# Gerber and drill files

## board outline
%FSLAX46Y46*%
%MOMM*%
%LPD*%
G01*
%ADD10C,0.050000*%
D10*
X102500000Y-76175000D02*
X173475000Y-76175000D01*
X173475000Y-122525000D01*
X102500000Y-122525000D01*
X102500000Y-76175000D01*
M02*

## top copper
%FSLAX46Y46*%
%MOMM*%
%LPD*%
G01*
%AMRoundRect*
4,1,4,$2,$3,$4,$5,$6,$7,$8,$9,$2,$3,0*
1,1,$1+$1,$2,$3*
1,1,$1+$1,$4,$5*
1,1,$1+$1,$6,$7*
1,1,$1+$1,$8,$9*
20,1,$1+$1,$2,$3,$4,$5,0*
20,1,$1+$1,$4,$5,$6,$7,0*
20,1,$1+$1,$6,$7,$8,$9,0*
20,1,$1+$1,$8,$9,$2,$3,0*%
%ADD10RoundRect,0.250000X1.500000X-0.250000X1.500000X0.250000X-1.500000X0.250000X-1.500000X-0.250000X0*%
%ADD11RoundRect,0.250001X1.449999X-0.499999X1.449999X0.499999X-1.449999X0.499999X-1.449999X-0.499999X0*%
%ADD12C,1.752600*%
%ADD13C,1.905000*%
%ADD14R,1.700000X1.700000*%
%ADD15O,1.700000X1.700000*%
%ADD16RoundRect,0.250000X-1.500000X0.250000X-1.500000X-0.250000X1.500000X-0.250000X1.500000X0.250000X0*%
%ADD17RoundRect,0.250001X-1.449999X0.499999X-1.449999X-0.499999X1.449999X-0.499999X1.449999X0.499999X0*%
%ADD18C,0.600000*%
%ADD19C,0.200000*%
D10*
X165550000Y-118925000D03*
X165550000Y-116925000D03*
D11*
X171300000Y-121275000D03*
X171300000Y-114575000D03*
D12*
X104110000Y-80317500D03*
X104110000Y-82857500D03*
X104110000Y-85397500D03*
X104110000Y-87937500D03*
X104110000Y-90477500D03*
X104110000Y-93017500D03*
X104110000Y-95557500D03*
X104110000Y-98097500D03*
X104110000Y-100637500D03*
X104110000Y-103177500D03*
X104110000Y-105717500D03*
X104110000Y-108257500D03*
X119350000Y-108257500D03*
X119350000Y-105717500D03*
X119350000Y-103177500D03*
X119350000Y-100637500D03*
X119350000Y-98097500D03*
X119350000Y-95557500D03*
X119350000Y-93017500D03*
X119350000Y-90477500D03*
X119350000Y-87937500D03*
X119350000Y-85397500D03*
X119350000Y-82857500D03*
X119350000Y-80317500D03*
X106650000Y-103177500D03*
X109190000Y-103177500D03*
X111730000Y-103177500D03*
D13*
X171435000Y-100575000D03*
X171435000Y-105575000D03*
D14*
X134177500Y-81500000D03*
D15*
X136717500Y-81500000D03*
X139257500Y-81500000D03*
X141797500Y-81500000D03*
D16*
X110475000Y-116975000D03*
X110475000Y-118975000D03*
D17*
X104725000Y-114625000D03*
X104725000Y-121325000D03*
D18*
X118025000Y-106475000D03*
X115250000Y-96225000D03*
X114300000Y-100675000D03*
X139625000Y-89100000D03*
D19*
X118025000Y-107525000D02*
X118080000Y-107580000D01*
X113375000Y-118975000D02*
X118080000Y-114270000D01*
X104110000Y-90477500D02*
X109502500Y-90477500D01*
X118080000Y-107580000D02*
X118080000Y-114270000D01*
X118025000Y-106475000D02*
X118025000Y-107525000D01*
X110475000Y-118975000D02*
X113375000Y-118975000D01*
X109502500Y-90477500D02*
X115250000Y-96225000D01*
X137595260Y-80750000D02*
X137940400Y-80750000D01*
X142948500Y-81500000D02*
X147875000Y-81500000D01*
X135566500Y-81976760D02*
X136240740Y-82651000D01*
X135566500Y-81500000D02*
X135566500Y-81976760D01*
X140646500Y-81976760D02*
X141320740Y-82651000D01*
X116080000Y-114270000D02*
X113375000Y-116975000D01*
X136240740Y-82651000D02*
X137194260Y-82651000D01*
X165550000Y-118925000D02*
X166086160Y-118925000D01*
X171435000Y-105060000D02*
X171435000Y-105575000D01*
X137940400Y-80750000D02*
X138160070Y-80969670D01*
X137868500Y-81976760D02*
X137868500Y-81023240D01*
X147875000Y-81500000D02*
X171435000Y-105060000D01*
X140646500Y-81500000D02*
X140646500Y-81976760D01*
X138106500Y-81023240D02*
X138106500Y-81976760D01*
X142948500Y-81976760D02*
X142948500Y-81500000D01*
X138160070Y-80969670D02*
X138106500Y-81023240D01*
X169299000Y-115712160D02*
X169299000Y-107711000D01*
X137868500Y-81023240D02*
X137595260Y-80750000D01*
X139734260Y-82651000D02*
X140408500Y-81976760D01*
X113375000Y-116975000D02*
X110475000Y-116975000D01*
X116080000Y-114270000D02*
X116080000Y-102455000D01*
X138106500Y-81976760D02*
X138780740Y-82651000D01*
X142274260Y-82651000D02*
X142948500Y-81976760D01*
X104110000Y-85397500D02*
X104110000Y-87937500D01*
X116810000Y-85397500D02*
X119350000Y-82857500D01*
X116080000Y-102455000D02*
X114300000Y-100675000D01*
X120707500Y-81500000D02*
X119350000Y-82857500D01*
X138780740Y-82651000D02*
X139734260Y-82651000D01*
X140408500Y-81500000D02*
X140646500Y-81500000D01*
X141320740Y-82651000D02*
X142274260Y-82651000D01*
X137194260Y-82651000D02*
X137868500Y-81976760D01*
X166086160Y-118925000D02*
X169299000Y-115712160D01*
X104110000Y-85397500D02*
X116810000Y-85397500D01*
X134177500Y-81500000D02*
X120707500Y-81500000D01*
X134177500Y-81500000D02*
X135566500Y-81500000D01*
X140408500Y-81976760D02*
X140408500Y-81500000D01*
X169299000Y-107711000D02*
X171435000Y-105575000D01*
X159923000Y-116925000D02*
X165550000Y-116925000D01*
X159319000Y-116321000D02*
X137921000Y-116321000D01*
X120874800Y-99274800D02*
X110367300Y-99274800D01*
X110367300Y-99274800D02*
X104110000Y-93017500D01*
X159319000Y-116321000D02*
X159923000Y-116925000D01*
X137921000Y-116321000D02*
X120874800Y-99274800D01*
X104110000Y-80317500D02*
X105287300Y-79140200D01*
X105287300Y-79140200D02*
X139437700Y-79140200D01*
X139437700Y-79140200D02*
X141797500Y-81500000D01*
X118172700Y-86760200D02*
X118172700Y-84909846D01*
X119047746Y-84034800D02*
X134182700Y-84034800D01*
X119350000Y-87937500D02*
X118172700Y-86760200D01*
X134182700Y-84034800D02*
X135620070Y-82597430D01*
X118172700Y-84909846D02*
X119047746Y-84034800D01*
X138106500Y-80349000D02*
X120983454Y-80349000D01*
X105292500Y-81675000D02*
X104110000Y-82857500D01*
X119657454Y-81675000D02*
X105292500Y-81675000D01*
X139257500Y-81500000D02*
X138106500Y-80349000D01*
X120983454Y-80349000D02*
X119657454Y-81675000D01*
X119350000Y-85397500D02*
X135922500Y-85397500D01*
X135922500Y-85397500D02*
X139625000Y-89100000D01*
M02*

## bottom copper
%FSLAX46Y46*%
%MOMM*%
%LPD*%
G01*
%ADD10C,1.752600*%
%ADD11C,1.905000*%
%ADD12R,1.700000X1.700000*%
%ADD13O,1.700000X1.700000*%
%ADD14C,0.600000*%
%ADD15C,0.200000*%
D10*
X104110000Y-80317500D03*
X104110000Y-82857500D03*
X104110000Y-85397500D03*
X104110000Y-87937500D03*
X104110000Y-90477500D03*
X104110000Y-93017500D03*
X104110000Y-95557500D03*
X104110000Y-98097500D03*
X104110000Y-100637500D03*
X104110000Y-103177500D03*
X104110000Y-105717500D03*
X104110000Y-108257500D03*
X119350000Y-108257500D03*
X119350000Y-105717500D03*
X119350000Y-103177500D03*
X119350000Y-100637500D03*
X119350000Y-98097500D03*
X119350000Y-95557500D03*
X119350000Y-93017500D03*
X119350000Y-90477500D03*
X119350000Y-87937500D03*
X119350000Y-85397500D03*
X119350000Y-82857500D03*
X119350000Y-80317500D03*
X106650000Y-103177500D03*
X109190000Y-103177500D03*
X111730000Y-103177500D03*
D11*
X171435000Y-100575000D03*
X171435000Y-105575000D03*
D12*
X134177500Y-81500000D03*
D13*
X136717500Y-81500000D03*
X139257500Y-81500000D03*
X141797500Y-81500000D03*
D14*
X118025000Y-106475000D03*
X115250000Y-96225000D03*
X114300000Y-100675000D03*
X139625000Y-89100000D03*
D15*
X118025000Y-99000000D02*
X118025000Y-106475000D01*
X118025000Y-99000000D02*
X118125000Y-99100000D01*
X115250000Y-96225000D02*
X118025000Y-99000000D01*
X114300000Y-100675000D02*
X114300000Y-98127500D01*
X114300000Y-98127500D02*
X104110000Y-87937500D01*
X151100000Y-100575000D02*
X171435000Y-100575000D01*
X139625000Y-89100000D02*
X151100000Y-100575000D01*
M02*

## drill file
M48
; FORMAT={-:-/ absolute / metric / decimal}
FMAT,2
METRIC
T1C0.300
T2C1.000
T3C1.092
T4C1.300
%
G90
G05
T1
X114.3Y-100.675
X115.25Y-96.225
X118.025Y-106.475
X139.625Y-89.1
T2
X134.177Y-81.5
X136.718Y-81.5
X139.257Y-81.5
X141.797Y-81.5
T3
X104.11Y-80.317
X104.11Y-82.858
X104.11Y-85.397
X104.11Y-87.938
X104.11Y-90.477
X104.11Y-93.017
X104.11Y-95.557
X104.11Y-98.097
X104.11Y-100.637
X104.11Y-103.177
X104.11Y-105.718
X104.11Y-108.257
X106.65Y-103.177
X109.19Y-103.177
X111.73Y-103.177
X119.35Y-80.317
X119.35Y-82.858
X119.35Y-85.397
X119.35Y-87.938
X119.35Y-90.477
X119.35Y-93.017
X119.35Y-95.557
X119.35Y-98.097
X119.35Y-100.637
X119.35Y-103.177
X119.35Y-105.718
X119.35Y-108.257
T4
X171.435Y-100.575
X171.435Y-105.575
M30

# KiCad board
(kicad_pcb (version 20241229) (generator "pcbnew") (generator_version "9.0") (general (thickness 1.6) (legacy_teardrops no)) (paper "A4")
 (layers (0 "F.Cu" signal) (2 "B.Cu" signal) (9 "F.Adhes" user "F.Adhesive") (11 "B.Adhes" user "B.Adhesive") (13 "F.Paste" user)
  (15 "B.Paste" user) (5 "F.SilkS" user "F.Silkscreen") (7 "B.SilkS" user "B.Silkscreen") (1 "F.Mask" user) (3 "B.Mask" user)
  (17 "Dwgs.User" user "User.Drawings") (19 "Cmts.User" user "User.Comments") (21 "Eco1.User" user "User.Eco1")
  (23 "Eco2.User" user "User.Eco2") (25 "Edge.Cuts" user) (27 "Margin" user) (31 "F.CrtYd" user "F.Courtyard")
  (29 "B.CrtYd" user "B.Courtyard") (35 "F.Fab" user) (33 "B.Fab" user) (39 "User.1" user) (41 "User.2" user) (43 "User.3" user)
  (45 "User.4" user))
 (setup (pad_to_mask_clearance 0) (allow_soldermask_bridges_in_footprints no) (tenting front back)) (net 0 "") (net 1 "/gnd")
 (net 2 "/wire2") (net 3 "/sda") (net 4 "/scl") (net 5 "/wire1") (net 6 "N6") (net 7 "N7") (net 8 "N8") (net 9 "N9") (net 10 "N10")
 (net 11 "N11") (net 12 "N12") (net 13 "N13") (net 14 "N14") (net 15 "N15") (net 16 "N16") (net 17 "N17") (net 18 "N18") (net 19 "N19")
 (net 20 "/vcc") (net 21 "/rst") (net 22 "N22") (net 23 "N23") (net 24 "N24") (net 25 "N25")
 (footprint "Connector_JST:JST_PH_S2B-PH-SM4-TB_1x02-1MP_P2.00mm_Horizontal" (layer "F.Cu") (at 168.4 117.925 90)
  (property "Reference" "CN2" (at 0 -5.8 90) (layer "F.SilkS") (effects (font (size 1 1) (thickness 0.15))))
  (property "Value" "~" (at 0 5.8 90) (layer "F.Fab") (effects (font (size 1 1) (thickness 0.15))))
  (pad "1" smd roundrect (at -1 -2.85 90) (size 1 3.5) (layers "F.Cu" "F.Mask" "F.Paste") (roundrect_rratio 0.25) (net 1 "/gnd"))
  (pad "2" smd roundrect (at 1 -2.85 90) (size 1 3.5) (layers "F.Cu" "F.Mask" "F.Paste") (roundrect_rratio 0.25) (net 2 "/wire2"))
  (pad "MP" smd roundrect (at -3.35 2.9 90) (size 1.5 3.4) (layers "F.Cu" "F.Mask" "F.Paste") (roundrect_rratio 0.166667))
  (pad "MP" smd roundrect (at 3.35 2.9 90) (size 1.5 3.4) (layers "F.Cu" "F.Mask" "F.Paste") (roundrect_rratio 0.166667)))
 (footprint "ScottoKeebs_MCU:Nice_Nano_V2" (layer "F.Cu") (at 111.73 94.0075)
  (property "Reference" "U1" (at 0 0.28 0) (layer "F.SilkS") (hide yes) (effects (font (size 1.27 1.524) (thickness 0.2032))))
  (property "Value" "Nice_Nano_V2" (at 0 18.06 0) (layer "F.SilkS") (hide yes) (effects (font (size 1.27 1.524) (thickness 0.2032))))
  (pad "1" thru_hole circle (at -7.62 -13.69 270) (size 1.7526 1.7526) (drill 1.0922) (layers "*.Cu" "*.Mask") (remove_unused_layers no)
   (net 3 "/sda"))
  (pad "2" thru_hole circle (at -7.62 -11.15 270) (size 1.7526 1.7526) (drill 1.0922) (layers "*.Cu" "*.Mask") (remove_unused_layers no)
   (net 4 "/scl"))
  (pad "3" thru_hole circle (at -7.62 -8.61 270) (size 1.7526 1.7526) (drill 1.0922) (layers "*.Cu" "*.Mask") (remove_unused_layers no)
   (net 1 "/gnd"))
  (pad "4" thru_hole circle (at -7.62 -6.07 270) (size 1.7526 1.7526) (drill 1.0922) (layers "*.Cu" "*.Mask") (remove_unused_layers no)
   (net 1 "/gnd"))
  (pad "5" thru_hole circle (at -7.62 -3.53 270) (size 1.7526 1.7526) (drill 1.0922) (layers "*.Cu" "*.Mask") (remove_unused_layers no)
   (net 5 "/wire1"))
  (pad "6" thru_hole circle (at -7.62 -0.99 270) (size 1.7526 1.7526) (drill 1.0922) (layers "*.Cu" "*.Mask") (remove_unused_layers no)
   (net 2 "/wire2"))
  (pad "7" thru_hole circle (at -7.62 1.55 270) (size 1.7526 1.7526) (drill 1.0922) (layers "*.Cu" "*.Mask") (remove_unused_layers no)
   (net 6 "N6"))
  (pad "8" thru_hole circle (at -7.62 4.09 270) (size 1.7526 1.7526) (drill 1.0922) (layers "*.Cu" "*.Mask") (remove_unused_layers no)
   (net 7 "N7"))
  (pad "9" thru_hole circle (at -7.62 6.63 270) (size 1.7526 1.7526) (drill 1.0922) (layers "*.Cu" "*.Mask") (remove_unused_layers no)
   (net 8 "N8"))
  (pad "10" thru_hole circle (at -7.62 9.17 270) (size 1.7526 1.7526) (drill 1.0922) (layers "*.Cu" "*.Mask") (remove_unused_layers no)
   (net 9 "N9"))
  (pad "11" thru_hole circle (at -7.62 11.71 270) (size 1.7526 1.7526) (drill 1.0922) (layers "*.Cu" "*.Mask") (remove_unused_layers no)
   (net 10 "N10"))
  (pad "12" thru_hole circle (at -7.62 14.25 270) (size 1.7526 1.7526) (drill 1.0922) (layers "*.Cu" "*.Mask") (remove_unused_layers no)
   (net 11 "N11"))
  (pad "13" thru_hole circle (at 7.62 14.25 270) (size 1.7526 1.7526) (drill 1.0922) (layers "*.Cu" "*.Mask") (remove_unused_layers no)
   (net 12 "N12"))
  (pad "14" thru_hole circle (at 7.62 11.71 270) (size 1.7526 1.7526) (drill 1.0922) (layers "*.Cu" "*.Mask") (remove_unused_layers no)
   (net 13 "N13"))
  (pad "15" thru_hole circle (at 7.62 9.17 270) (size 1.7526 1.7526) (drill 1.0922) (layers "*.Cu" "*.Mask") (remove_unused_layers no)
   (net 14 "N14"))
  (pad "16" thru_hole circle (at 7.62 6.63 270) (size 1.7526 1.7526) (drill 1.0922) (layers "*.Cu" "*.Mask") (remove_unused_layers no)
   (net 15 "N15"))
  (pad "17" thru_hole circle (at 7.62 4.09 270) (size 1.7526 1.7526) (drill 1.0922) (layers "*.Cu" "*.Mask") (remove_unused_layers no)
   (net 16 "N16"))
  (pad "18" thru_hole circle (at 7.62 1.55 270) (size 1.7526 1.7526) (drill 1.0922) (layers "*.Cu" "*.Mask") (remove_unused_layers no)
   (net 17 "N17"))
  (pad "19" thru_hole circle (at 7.62 -0.99 270) (size 1.7526 1.7526) (drill 1.0922) (layers "*.Cu" "*.Mask") (remove_unused_layers no)
   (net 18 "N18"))
  (pad "20" thru_hole circle (at 7.62 -3.53 270) (size 1.7526 1.7526) (drill 1.0922) (layers "*.Cu" "*.Mask") (remove_unused_layers no)
   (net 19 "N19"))
  (pad "21" thru_hole circle (at 7.62 -6.07 270) (size 1.7526 1.7526) (drill 1.0922) (layers "*.Cu" "*.Mask") (remove_unused_layers no)
   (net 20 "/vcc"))
  (pad "22" thru_hole circle (at 7.62 -8.61 270) (size 1.7526 1.7526) (drill 1.0922) (layers "*.Cu" "*.Mask") (remove_unused_layers no)
   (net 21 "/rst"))
  (pad "23" thru_hole circle (at 7.62 -11.15 270) (size 1.7526 1.7526) (drill 1.0922) (layers "*.Cu" "*.Mask") (remove_unused_layers no)
   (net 1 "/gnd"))
  (pad "24" thru_hole circle (at 7.62 -13.69 270) (size 1.7526 1.7526) (drill 1.0922) (layers "*.Cu" "*.Mask") (remove_unused_layers no)
   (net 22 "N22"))
  (pad "25" thru_hole circle (at -5.08 9.17) (size 1.7526 1.7526) (drill 1.0922) (layers "*.Cu" "*.Mask") (remove_unused_layers no)
   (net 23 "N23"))
  (pad "26" thru_hole circle (at -2.54 9.17) (size 1.7526 1.7526) (drill 1.0922) (layers "*.Cu" "*.Mask") (remove_unused_layers no)
   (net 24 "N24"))
  (pad "27" thru_hole circle (at 0 9.17) (size 1.7526 1.7526) (drill 1.0922) (layers "*.Cu" "*.Mask") (remove_unused_layers no)
   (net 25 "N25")))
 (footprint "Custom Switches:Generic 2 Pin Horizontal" (layer "F.Cu") (at 171.435 103.075 -90)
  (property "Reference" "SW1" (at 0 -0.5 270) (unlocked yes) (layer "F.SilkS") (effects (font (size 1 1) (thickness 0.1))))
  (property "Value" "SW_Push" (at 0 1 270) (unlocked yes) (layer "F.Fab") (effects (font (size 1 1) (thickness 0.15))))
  (pad "1" thru_hole circle (at -2.5 0 270) (size 1.905 1.905) (drill 1.3) (layers "*.Cu" "*.Mask") (remove_unused_layers no)
   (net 21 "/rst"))
  (pad "2" thru_hole circle (at 2.5 0 270) (size 1.905 1.905) (drill 1.3) (layers "*.Cu" "*.Mask") (remove_unused_layers no) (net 1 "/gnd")))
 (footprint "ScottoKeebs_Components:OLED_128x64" (layer "F.Cu") (at 137.9875 81.5)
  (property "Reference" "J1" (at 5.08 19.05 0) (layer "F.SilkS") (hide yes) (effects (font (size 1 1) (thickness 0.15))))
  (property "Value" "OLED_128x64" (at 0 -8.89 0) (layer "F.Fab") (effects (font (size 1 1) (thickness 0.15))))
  (pad "1" thru_hole rect (at -3.81 0 90) (size 1.7 1.7) (drill 1) (layers "*.Cu" "*.Mask") (remove_unused_layers no) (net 1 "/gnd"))
  (pad "2" thru_hole oval (at -1.27 0 90) (size 1.7 1.7) (drill 1) (layers "*.Cu" "*.Mask") (remove_unused_layers no) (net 20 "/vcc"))
  (pad "3" thru_hole oval (at 1.27 0 90) (size 1.7 1.7) (drill 1) (layers "*.Cu" "*.Mask") (remove_unused_layers no) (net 4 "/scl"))
  (pad "4" thru_hole oval (at 3.81 0 90) (size 1.7 1.7) (drill 1) (layers "*.Cu" "*.Mask") (remove_unused_layers no) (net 3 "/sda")))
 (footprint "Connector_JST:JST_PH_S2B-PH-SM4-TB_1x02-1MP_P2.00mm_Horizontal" (layer "F.Cu") (at 107.625 117.975 -90)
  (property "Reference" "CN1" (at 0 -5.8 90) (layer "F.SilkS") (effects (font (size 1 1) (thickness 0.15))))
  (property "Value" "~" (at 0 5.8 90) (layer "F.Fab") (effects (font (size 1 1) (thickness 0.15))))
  (pad "1" smd roundrect (at -1 -2.85 270) (size 1 3.5) (layers "F.Cu" "F.Mask" "F.Paste") (roundrect_rratio 0.25) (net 1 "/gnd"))
  (pad "2" smd roundrect (at 1 -2.85 270) (size 1 3.5) (layers "F.Cu" "F.Mask" "F.Paste") (roundrect_rratio 0.25) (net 5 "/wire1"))
  (pad "MP" smd roundrect (at -3.35 2.9 270) (size 1.5 3.4) (layers "F.Cu" "F.Mask" "F.Paste") (roundrect_rratio 0.166667))
  (pad "MP" smd roundrect (at 3.35 2.9 270) (size 1.5 3.4) (layers "F.Cu" "F.Mask" "F.Paste") (roundrect_rratio 0.166667)))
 (gr_rect (start 102.5 76.175) (end 173.475 122.525) (stroke (width 0.05) (type default)) (fill no) (layer "Edge.Cuts"))
 (segment (start 118.025 107.525) (end 118.08 107.58) (width 0.2) (layer "F.Cu") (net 5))
 (segment (start 113.375 118.975) (end 118.08 114.27) (width 0.2) (layer "F.Cu") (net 5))
 (segment (start 104.11 90.4775) (end 109.5025 90.4775) (width 0.2) (layer "F.Cu") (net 5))
 (segment (start 118.08 107.58) (end 118.08 114.27) (width 0.2) (layer "F.Cu") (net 5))
 (segment (start 118.025 106.475) (end 118.025 107.525) (width 0.2) (layer "F.Cu") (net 5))
 (segment (start 110.475 118.975) (end 113.375 118.975) (width 0.2) (layer "F.Cu") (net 5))
 (segment (start 109.5025 90.4775) (end 115.25 96.225) (width 0.2) (layer "F.Cu") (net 5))
 (via (at 118.025 106.475) (size 0.6) (drill 0.3) (layers "F.Cu" "B.Cu") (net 5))
 (via (at 115.25 96.225) (size 0.6) (drill 0.3) (layers "F.Cu" "B.Cu") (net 5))
 (segment (start 118.025 99) (end 118.025 106.475) (width 0.2) (layer "B.Cu") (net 5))
 (segment (start 118.025 99) (end 118.125 99.1) (width 0.2) (layer "B.Cu") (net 5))
 (segment (start 115.25 96.225) (end 118.025 99) (width 0.2) (layer "B.Cu") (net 5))
 (segment (start 137.59526 80.75) (end 137.9404 80.75) (width 0.2) (layer "F.Cu") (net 1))
 (segment (start 142.9485 81.5) (end 147.875 81.5) (width 0.2) (layer "F.Cu") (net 1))
 (segment (start 135.5665 81.97676) (end 136.24074 82.651) (width 0.2) (layer "F.Cu") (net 1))
 (segment (start 135.5665 81.5) (end 135.5665 81.97676) (width 0.2) (layer "F.Cu") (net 1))
 (segment (start 140.6465 81.97676) (end 141.32074 82.651) (width 0.2) (layer "F.Cu") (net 1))
 (segment (start 116.08 114.27) (end 113.375 116.975) (width 0.2) (layer "F.Cu") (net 1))
 (segment (start 136.24074 82.651) (end 137.19426 82.651) (width 0.2) (layer "F.Cu") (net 1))
 (segment (start 165.55 118.925) (end 166.08616 118.925) (width 0.2) (layer "F.Cu") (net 1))
 (segment (start 171.435 105.06) (end 171.435 105.575) (width 0.2) (layer "F.Cu") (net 1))
 (segment (start 137.9404 80.75) (end 138.16007 80.96967) (width 0.2) (layer "F.Cu") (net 1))
 (segment (start 137.8685 81.97676) (end 137.8685 81.02324) (width 0.2) (layer "F.Cu") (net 1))
 (segment (start 147.875 81.5) (end 171.435 105.06) (width 0.2) (layer "F.Cu") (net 1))
 (segment (start 140.6465 81.5) (end 140.6465 81.97676) (width 0.2) (layer "F.Cu") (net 1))
 (segment (start 138.1065 81.02324) (end 138.1065 81.97676) (width 0.2) (layer "F.Cu") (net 1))
 (segment (start 142.9485 81.97676) (end 142.9485 81.5) (width 0.2) (layer "F.Cu") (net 1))
 (segment (start 138.16007 80.96967) (end 138.1065 81.02324) (width 0.2) (layer "F.Cu") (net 1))
 (segment (start 169.299 115.71216) (end 169.299 107.711) (width 0.2) (layer "F.Cu") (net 1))
 (segment (start 137.8685 81.02324) (end 137.59526 80.75) (width 0.2) (layer "F.Cu") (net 1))
 (segment (start 139.73426 82.651) (end 140.4085 81.97676) (width 0.2) (layer "F.Cu") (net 1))
 (segment (start 113.375 116.975) (end 110.475 116.975) (width 0.2) (layer "F.Cu") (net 1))
 (segment (start 116.08 114.27) (end 116.08 102.455) (width 0.2) (layer "F.Cu") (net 1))
 (segment (start 138.1065 81.97676) (end 138.78074 82.651) (width 0.2) (layer "F.Cu") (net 1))
 (segment (start 142.27426 82.651) (end 142.9485 81.97676) (width 0.2) (layer "F.Cu") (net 1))
 (segment (start 104.11 85.3975) (end 104.11 87.9375) (width 0.2) (layer "F.Cu") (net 1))
 (segment (start 116.81 85.3975) (end 119.35 82.8575) (width 0.2) (layer "F.Cu") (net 1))
 (segment (start 116.08 102.455) (end 114.3 100.675) (width 0.2) (layer "F.Cu") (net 1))
 (segment (start 120.7075 81.5) (end 119.35 82.8575) (width 0.2) (layer "F.Cu") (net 1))
 (segment (start 138.78074 82.651) (end 139.73426 82.651) (width 0.2) (layer "F.Cu") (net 1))
 (segment (start 140.4085 81.5) (end 140.6465 81.5) (width 0.2) (layer "F.Cu") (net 1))
 (segment (start 141.32074 82.651) (end 142.27426 82.651) (width 0.2) (layer "F.Cu") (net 1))
 (segment (start 137.19426 82.651) (end 137.8685 81.97676) (width 0.2) (layer "F.Cu") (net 1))
 (segment (start 166.08616 118.925) (end 169.299 115.71216) (width 0.2) (layer "F.Cu") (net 1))
 (segment (start 104.11 85.3975) (end 116.81 85.3975) (width 0.2) (layer "F.Cu") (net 1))
 (segment (start 134.1775 81.5) (end 120.7075 81.5) (width 0.2) (layer "F.Cu") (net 1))
 (segment (start 134.1775 81.5) (end 135.5665 81.5) (width 0.2) (layer "F.Cu") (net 1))
 (segment (start 140.4085 81.97676) (end 140.4085 81.5) (width 0.2) (layer "F.Cu") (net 1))
 (segment (start 169.299 107.711) (end 171.435 105.575) (width 0.2) (layer "F.Cu") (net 1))
 (via (at 114.3 100.675) (size 0.6) (drill 0.3) (layers "F.Cu" "B.Cu") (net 1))
 (segment (start 114.3 100.675) (end 114.3 98.1275) (width 0.2) (layer "B.Cu") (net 1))
 (segment (start 114.3 98.1275) (end 104.11 87.9375) (width 0.2) (layer "B.Cu") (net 1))
 (segment (start 159.923 116.925) (end 165.55 116.925) (width 0.2) (layer "F.Cu") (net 2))
 (segment (start 159.319 116.321) (end 137.921 116.321) (width 0.2) (layer "F.Cu") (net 2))
 (segment (start 120.8748 99.2748) (end 110.3673 99.2748) (width 0.2) (layer "F.Cu") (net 2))
 (segment (start 110.3673 99.2748) (end 104.11 93.0175) (width 0.2) (layer "F.Cu") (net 2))
 (segment (start 159.319 116.321) (end 159.923 116.925) (width 0.2) (layer "F.Cu") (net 2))
 (segment (start 137.921 116.321) (end 120.8748 99.2748) (width 0.2) (layer "F.Cu") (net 2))
 (segment (start 104.11 80.3175) (end 105.2873 79.1402) (width 0.2) (layer "F.Cu") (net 3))
 (segment (start 105.2873 79.1402) (end 139.4377 79.1402) (width 0.2) (layer "F.Cu") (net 3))
 (segment (start 139.4377 79.1402) (end 141.7975 81.5) (width 0.2) (layer "F.Cu") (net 3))
 (segment (start 118.1727 86.7602) (end 118.1727 84.909846) (width 0.2) (layer "F.Cu") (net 20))
 (segment (start 119.047746 84.0348) (end 134.1827 84.0348) (width 0.2) (layer "F.Cu") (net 20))
 (segment (start 119.35 87.9375) (end 118.1727 86.7602) (width 0.2) (layer "F.Cu") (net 20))
 (segment (start 134.1827 84.0348) (end 135.62007 82.59743) (width 0.2) (layer "F.Cu") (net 20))
 (segment (start 118.1727 84.909846) (end 119.047746 84.0348) (width 0.2) (layer "F.Cu") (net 20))
 (segment (start 138.1065 80.349) (end 120.983454 80.349) (width 0.2) (layer "F.Cu") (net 4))
 (segment (start 105.2925 81.675) (end 104.11 82.8575) (width 0.2) (layer "F.Cu") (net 4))
 (segment (start 119.657454 81.675) (end 105.2925 81.675) (width 0.2) (layer "F.Cu") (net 4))
 (segment (start 139.2575 81.5) (end 138.1065 80.349) (width 0.2) (layer "F.Cu") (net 4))
 (segment (start 120.983454 80.349) (end 119.657454 81.675) (width 0.2) (layer "F.Cu") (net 4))
 (segment (start 119.35 85.3975) (end 135.9225 85.3975) (width 0.2) (layer "F.Cu") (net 21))
 (segment (start 135.9225 85.3975) (end 139.625 89.1) (width 0.2) (layer "F.Cu") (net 21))
 (via (at 139.625 89.1) (size 0.6) (drill 0.3) (layers "F.Cu" "B.Cu") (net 21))
 (segment (start 151.1 100.575) (end 171.435 100.575) (width 0.2) (layer "B.Cu") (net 21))
 (segment (start 139.625 89.1) (end 151.1 100.575) (width 0.2) (layer "B.Cu") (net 21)))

